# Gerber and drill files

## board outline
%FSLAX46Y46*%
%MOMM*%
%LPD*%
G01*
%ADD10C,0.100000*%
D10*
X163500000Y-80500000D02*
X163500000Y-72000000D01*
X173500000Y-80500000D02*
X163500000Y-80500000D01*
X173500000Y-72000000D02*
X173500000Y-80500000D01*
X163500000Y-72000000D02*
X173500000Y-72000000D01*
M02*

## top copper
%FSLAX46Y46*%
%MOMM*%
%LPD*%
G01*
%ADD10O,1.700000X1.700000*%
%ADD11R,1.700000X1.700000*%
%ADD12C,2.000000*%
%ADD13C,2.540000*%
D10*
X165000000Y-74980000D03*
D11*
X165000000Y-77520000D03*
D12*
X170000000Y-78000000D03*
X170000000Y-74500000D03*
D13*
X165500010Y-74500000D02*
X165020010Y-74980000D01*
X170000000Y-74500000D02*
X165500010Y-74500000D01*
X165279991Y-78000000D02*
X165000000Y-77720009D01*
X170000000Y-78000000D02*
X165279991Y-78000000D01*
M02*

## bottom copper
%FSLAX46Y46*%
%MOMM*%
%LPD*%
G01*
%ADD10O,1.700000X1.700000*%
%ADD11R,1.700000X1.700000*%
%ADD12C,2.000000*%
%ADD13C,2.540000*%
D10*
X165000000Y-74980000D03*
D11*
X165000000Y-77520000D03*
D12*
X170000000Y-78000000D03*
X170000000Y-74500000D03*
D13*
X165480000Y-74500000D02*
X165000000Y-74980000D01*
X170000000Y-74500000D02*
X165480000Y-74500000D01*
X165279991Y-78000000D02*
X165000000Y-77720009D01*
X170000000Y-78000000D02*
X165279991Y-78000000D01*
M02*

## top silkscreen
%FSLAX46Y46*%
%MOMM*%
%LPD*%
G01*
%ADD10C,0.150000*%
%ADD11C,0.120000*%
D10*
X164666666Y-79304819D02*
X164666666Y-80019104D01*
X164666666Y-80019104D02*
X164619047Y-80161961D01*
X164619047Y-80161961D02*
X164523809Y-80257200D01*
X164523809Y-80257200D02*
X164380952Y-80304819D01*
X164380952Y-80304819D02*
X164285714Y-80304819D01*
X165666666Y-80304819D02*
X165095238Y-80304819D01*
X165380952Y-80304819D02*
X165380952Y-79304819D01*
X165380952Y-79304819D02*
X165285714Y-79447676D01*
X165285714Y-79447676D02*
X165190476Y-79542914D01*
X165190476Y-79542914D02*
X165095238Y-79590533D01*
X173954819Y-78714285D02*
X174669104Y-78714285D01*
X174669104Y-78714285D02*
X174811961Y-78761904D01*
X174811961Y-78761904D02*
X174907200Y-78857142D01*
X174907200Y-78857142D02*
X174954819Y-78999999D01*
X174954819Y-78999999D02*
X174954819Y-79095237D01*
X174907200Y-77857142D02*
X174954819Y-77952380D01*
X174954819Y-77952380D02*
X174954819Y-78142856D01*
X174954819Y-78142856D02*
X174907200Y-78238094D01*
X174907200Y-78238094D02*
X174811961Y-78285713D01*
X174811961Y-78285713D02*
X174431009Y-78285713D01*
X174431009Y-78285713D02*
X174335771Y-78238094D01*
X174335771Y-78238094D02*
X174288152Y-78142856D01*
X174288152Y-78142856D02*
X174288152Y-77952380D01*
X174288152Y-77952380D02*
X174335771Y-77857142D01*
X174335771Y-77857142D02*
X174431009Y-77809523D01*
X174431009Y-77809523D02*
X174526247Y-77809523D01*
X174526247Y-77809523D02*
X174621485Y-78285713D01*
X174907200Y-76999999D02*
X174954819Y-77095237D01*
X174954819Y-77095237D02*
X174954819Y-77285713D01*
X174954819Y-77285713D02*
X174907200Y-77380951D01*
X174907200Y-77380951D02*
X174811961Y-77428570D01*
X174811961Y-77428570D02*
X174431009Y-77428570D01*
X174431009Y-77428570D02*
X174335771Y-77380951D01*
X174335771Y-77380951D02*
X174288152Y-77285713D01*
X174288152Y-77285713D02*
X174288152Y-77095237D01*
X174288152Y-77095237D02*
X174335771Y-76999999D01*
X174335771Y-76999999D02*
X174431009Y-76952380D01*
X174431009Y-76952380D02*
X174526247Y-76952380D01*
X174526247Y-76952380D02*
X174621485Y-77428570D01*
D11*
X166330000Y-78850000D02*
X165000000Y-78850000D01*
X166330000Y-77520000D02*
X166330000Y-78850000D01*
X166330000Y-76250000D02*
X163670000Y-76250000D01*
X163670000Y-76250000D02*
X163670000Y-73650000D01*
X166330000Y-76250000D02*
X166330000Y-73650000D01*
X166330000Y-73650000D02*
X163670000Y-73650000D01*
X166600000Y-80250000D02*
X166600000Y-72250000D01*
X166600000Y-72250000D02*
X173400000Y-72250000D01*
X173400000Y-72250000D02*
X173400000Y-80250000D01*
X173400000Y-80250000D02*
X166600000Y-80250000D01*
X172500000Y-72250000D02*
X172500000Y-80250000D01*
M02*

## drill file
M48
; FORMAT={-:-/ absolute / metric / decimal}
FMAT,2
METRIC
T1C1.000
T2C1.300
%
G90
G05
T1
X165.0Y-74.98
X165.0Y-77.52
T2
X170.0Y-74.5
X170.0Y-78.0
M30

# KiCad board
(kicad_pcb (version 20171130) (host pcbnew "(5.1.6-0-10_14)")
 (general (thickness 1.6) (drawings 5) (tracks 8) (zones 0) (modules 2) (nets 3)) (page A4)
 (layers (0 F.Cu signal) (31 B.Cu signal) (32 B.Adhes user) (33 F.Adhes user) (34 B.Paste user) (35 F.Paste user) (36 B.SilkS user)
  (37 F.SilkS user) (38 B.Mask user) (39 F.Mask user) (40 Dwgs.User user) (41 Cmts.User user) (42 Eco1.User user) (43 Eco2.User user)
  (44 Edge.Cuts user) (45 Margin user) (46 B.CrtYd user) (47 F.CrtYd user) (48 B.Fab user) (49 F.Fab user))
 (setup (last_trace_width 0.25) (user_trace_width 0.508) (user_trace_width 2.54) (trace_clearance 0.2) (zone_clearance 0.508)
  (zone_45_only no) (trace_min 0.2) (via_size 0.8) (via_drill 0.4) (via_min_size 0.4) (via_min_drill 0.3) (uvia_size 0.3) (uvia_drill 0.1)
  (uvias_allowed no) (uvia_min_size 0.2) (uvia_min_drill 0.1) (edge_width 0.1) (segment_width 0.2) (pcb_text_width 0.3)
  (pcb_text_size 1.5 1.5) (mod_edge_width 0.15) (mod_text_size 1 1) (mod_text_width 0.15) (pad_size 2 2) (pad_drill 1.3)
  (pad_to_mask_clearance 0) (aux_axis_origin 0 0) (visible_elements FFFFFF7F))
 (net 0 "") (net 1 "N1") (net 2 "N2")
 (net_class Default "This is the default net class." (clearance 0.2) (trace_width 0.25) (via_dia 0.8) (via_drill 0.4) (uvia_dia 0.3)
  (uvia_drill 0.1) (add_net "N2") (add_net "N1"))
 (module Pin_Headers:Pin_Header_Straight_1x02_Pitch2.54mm (layer F.Cu) (at 165 77.52 180)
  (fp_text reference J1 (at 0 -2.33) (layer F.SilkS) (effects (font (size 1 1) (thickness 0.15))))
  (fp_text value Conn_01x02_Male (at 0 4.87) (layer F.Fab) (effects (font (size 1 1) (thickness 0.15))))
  (fp_line (start -1.33 -1.33) (end 0 -1.33) (layer F.SilkS) (width 0.12))
  (fp_line (start -1.33 0) (end -1.33 -1.33) (layer F.SilkS) (width 0.12))
  (fp_line (start -1.33 1.27) (end 1.33 1.27) (layer F.SilkS) (width 0.12))
  (fp_line (start 1.33 1.27) (end 1.33 3.87) (layer F.SilkS) (width 0.12))
  (fp_line (start -1.33 1.27) (end -1.33 3.87) (layer F.SilkS) (width 0.12))
  (fp_line (start -1.33 3.87) (end 1.33 3.87) (layer F.SilkS) (width 0.12))
  (pad 2 thru_hole oval (at 0 2.54 180) (size 1.7 1.7) (drill 1) (layers *.Cu *.Mask) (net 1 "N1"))
  (pad 1 thru_hole rect (at 0 0 180) (size 1.7 1.7) (drill 1) (layers *.Cu *.Mask) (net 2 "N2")))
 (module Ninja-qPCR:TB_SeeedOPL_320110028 (layer F.Cu) (at 170 78 90)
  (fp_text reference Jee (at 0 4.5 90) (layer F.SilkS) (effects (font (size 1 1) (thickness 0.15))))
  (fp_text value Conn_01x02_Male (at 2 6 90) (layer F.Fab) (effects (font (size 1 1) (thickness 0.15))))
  (fp_line (start -2.25 -3.4) (end 5.75 -3.4) (layer F.SilkS) (width 0.12))
  (fp_line (start 5.75 -3.4) (end 5.75 3.4) (layer F.SilkS) (width 0.12))
  (fp_line (start 5.75 3.4) (end -2.25 3.4) (layer F.SilkS) (width 0.12))
  (fp_line (start -2.25 3.4) (end -2.25 -3.4) (layer F.SilkS) (width 0.12))
  (fp_line (start 5.75 2.5) (end -2.25 2.5) (layer F.SilkS) (width 0.12))
  (pad 1 thru_hole circle (at 0 0 90) (size 2 2) (drill 1.3) (layers *.Cu *.Mask) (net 2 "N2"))
  (pad 2 thru_hole circle (at 3.5 0 90) (size 2 2) (drill 1.3) (layers *.Cu *.Mask) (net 1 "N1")))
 (gr_line (start 163.5 80.5) (end 163.5 72) (layer Edge.Cuts) (width 0.1))
 (gr_line (start 173.5 80.5) (end 163.5 80.5) (layer Edge.Cuts) (width 0.1))
 (gr_line (start 173.5 72) (end 173.5 80.5) (layer Edge.Cuts) (width 0.1))
 (gr_line (start 163.5 72) (end 173.5 72) (layer Edge.Cuts) (width 0.1))
 (segment (start 165.48 74.5) (end 165 74.98) (width 2.54) (layer B.Cu) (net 1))
 (segment (start 170 74.5) (end 165.48 74.5) (width 2.54) (layer B.Cu) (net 1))
 (segment (start 165.50001 74.5) (end 165.02001 74.98) (width 2.54) (layer F.Cu) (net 1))
 (segment (start 170 74.5) (end 165.50001 74.5) (width 2.54) (layer F.Cu) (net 1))
 (segment (start 165.279991 78) (end 165 77.720009) (width 2.54) (layer F.Cu) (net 2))
 (segment (start 170 78) (end 165.279991 78) (width 2.54) (layer F.Cu) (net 2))
 (segment (start 165.279991 78) (end 165 77.720009) (width 2.54) (layer B.Cu) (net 2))
 (segment (start 170 78) (end 165.279991 78) (width 2.54) (layer B.Cu) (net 2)))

